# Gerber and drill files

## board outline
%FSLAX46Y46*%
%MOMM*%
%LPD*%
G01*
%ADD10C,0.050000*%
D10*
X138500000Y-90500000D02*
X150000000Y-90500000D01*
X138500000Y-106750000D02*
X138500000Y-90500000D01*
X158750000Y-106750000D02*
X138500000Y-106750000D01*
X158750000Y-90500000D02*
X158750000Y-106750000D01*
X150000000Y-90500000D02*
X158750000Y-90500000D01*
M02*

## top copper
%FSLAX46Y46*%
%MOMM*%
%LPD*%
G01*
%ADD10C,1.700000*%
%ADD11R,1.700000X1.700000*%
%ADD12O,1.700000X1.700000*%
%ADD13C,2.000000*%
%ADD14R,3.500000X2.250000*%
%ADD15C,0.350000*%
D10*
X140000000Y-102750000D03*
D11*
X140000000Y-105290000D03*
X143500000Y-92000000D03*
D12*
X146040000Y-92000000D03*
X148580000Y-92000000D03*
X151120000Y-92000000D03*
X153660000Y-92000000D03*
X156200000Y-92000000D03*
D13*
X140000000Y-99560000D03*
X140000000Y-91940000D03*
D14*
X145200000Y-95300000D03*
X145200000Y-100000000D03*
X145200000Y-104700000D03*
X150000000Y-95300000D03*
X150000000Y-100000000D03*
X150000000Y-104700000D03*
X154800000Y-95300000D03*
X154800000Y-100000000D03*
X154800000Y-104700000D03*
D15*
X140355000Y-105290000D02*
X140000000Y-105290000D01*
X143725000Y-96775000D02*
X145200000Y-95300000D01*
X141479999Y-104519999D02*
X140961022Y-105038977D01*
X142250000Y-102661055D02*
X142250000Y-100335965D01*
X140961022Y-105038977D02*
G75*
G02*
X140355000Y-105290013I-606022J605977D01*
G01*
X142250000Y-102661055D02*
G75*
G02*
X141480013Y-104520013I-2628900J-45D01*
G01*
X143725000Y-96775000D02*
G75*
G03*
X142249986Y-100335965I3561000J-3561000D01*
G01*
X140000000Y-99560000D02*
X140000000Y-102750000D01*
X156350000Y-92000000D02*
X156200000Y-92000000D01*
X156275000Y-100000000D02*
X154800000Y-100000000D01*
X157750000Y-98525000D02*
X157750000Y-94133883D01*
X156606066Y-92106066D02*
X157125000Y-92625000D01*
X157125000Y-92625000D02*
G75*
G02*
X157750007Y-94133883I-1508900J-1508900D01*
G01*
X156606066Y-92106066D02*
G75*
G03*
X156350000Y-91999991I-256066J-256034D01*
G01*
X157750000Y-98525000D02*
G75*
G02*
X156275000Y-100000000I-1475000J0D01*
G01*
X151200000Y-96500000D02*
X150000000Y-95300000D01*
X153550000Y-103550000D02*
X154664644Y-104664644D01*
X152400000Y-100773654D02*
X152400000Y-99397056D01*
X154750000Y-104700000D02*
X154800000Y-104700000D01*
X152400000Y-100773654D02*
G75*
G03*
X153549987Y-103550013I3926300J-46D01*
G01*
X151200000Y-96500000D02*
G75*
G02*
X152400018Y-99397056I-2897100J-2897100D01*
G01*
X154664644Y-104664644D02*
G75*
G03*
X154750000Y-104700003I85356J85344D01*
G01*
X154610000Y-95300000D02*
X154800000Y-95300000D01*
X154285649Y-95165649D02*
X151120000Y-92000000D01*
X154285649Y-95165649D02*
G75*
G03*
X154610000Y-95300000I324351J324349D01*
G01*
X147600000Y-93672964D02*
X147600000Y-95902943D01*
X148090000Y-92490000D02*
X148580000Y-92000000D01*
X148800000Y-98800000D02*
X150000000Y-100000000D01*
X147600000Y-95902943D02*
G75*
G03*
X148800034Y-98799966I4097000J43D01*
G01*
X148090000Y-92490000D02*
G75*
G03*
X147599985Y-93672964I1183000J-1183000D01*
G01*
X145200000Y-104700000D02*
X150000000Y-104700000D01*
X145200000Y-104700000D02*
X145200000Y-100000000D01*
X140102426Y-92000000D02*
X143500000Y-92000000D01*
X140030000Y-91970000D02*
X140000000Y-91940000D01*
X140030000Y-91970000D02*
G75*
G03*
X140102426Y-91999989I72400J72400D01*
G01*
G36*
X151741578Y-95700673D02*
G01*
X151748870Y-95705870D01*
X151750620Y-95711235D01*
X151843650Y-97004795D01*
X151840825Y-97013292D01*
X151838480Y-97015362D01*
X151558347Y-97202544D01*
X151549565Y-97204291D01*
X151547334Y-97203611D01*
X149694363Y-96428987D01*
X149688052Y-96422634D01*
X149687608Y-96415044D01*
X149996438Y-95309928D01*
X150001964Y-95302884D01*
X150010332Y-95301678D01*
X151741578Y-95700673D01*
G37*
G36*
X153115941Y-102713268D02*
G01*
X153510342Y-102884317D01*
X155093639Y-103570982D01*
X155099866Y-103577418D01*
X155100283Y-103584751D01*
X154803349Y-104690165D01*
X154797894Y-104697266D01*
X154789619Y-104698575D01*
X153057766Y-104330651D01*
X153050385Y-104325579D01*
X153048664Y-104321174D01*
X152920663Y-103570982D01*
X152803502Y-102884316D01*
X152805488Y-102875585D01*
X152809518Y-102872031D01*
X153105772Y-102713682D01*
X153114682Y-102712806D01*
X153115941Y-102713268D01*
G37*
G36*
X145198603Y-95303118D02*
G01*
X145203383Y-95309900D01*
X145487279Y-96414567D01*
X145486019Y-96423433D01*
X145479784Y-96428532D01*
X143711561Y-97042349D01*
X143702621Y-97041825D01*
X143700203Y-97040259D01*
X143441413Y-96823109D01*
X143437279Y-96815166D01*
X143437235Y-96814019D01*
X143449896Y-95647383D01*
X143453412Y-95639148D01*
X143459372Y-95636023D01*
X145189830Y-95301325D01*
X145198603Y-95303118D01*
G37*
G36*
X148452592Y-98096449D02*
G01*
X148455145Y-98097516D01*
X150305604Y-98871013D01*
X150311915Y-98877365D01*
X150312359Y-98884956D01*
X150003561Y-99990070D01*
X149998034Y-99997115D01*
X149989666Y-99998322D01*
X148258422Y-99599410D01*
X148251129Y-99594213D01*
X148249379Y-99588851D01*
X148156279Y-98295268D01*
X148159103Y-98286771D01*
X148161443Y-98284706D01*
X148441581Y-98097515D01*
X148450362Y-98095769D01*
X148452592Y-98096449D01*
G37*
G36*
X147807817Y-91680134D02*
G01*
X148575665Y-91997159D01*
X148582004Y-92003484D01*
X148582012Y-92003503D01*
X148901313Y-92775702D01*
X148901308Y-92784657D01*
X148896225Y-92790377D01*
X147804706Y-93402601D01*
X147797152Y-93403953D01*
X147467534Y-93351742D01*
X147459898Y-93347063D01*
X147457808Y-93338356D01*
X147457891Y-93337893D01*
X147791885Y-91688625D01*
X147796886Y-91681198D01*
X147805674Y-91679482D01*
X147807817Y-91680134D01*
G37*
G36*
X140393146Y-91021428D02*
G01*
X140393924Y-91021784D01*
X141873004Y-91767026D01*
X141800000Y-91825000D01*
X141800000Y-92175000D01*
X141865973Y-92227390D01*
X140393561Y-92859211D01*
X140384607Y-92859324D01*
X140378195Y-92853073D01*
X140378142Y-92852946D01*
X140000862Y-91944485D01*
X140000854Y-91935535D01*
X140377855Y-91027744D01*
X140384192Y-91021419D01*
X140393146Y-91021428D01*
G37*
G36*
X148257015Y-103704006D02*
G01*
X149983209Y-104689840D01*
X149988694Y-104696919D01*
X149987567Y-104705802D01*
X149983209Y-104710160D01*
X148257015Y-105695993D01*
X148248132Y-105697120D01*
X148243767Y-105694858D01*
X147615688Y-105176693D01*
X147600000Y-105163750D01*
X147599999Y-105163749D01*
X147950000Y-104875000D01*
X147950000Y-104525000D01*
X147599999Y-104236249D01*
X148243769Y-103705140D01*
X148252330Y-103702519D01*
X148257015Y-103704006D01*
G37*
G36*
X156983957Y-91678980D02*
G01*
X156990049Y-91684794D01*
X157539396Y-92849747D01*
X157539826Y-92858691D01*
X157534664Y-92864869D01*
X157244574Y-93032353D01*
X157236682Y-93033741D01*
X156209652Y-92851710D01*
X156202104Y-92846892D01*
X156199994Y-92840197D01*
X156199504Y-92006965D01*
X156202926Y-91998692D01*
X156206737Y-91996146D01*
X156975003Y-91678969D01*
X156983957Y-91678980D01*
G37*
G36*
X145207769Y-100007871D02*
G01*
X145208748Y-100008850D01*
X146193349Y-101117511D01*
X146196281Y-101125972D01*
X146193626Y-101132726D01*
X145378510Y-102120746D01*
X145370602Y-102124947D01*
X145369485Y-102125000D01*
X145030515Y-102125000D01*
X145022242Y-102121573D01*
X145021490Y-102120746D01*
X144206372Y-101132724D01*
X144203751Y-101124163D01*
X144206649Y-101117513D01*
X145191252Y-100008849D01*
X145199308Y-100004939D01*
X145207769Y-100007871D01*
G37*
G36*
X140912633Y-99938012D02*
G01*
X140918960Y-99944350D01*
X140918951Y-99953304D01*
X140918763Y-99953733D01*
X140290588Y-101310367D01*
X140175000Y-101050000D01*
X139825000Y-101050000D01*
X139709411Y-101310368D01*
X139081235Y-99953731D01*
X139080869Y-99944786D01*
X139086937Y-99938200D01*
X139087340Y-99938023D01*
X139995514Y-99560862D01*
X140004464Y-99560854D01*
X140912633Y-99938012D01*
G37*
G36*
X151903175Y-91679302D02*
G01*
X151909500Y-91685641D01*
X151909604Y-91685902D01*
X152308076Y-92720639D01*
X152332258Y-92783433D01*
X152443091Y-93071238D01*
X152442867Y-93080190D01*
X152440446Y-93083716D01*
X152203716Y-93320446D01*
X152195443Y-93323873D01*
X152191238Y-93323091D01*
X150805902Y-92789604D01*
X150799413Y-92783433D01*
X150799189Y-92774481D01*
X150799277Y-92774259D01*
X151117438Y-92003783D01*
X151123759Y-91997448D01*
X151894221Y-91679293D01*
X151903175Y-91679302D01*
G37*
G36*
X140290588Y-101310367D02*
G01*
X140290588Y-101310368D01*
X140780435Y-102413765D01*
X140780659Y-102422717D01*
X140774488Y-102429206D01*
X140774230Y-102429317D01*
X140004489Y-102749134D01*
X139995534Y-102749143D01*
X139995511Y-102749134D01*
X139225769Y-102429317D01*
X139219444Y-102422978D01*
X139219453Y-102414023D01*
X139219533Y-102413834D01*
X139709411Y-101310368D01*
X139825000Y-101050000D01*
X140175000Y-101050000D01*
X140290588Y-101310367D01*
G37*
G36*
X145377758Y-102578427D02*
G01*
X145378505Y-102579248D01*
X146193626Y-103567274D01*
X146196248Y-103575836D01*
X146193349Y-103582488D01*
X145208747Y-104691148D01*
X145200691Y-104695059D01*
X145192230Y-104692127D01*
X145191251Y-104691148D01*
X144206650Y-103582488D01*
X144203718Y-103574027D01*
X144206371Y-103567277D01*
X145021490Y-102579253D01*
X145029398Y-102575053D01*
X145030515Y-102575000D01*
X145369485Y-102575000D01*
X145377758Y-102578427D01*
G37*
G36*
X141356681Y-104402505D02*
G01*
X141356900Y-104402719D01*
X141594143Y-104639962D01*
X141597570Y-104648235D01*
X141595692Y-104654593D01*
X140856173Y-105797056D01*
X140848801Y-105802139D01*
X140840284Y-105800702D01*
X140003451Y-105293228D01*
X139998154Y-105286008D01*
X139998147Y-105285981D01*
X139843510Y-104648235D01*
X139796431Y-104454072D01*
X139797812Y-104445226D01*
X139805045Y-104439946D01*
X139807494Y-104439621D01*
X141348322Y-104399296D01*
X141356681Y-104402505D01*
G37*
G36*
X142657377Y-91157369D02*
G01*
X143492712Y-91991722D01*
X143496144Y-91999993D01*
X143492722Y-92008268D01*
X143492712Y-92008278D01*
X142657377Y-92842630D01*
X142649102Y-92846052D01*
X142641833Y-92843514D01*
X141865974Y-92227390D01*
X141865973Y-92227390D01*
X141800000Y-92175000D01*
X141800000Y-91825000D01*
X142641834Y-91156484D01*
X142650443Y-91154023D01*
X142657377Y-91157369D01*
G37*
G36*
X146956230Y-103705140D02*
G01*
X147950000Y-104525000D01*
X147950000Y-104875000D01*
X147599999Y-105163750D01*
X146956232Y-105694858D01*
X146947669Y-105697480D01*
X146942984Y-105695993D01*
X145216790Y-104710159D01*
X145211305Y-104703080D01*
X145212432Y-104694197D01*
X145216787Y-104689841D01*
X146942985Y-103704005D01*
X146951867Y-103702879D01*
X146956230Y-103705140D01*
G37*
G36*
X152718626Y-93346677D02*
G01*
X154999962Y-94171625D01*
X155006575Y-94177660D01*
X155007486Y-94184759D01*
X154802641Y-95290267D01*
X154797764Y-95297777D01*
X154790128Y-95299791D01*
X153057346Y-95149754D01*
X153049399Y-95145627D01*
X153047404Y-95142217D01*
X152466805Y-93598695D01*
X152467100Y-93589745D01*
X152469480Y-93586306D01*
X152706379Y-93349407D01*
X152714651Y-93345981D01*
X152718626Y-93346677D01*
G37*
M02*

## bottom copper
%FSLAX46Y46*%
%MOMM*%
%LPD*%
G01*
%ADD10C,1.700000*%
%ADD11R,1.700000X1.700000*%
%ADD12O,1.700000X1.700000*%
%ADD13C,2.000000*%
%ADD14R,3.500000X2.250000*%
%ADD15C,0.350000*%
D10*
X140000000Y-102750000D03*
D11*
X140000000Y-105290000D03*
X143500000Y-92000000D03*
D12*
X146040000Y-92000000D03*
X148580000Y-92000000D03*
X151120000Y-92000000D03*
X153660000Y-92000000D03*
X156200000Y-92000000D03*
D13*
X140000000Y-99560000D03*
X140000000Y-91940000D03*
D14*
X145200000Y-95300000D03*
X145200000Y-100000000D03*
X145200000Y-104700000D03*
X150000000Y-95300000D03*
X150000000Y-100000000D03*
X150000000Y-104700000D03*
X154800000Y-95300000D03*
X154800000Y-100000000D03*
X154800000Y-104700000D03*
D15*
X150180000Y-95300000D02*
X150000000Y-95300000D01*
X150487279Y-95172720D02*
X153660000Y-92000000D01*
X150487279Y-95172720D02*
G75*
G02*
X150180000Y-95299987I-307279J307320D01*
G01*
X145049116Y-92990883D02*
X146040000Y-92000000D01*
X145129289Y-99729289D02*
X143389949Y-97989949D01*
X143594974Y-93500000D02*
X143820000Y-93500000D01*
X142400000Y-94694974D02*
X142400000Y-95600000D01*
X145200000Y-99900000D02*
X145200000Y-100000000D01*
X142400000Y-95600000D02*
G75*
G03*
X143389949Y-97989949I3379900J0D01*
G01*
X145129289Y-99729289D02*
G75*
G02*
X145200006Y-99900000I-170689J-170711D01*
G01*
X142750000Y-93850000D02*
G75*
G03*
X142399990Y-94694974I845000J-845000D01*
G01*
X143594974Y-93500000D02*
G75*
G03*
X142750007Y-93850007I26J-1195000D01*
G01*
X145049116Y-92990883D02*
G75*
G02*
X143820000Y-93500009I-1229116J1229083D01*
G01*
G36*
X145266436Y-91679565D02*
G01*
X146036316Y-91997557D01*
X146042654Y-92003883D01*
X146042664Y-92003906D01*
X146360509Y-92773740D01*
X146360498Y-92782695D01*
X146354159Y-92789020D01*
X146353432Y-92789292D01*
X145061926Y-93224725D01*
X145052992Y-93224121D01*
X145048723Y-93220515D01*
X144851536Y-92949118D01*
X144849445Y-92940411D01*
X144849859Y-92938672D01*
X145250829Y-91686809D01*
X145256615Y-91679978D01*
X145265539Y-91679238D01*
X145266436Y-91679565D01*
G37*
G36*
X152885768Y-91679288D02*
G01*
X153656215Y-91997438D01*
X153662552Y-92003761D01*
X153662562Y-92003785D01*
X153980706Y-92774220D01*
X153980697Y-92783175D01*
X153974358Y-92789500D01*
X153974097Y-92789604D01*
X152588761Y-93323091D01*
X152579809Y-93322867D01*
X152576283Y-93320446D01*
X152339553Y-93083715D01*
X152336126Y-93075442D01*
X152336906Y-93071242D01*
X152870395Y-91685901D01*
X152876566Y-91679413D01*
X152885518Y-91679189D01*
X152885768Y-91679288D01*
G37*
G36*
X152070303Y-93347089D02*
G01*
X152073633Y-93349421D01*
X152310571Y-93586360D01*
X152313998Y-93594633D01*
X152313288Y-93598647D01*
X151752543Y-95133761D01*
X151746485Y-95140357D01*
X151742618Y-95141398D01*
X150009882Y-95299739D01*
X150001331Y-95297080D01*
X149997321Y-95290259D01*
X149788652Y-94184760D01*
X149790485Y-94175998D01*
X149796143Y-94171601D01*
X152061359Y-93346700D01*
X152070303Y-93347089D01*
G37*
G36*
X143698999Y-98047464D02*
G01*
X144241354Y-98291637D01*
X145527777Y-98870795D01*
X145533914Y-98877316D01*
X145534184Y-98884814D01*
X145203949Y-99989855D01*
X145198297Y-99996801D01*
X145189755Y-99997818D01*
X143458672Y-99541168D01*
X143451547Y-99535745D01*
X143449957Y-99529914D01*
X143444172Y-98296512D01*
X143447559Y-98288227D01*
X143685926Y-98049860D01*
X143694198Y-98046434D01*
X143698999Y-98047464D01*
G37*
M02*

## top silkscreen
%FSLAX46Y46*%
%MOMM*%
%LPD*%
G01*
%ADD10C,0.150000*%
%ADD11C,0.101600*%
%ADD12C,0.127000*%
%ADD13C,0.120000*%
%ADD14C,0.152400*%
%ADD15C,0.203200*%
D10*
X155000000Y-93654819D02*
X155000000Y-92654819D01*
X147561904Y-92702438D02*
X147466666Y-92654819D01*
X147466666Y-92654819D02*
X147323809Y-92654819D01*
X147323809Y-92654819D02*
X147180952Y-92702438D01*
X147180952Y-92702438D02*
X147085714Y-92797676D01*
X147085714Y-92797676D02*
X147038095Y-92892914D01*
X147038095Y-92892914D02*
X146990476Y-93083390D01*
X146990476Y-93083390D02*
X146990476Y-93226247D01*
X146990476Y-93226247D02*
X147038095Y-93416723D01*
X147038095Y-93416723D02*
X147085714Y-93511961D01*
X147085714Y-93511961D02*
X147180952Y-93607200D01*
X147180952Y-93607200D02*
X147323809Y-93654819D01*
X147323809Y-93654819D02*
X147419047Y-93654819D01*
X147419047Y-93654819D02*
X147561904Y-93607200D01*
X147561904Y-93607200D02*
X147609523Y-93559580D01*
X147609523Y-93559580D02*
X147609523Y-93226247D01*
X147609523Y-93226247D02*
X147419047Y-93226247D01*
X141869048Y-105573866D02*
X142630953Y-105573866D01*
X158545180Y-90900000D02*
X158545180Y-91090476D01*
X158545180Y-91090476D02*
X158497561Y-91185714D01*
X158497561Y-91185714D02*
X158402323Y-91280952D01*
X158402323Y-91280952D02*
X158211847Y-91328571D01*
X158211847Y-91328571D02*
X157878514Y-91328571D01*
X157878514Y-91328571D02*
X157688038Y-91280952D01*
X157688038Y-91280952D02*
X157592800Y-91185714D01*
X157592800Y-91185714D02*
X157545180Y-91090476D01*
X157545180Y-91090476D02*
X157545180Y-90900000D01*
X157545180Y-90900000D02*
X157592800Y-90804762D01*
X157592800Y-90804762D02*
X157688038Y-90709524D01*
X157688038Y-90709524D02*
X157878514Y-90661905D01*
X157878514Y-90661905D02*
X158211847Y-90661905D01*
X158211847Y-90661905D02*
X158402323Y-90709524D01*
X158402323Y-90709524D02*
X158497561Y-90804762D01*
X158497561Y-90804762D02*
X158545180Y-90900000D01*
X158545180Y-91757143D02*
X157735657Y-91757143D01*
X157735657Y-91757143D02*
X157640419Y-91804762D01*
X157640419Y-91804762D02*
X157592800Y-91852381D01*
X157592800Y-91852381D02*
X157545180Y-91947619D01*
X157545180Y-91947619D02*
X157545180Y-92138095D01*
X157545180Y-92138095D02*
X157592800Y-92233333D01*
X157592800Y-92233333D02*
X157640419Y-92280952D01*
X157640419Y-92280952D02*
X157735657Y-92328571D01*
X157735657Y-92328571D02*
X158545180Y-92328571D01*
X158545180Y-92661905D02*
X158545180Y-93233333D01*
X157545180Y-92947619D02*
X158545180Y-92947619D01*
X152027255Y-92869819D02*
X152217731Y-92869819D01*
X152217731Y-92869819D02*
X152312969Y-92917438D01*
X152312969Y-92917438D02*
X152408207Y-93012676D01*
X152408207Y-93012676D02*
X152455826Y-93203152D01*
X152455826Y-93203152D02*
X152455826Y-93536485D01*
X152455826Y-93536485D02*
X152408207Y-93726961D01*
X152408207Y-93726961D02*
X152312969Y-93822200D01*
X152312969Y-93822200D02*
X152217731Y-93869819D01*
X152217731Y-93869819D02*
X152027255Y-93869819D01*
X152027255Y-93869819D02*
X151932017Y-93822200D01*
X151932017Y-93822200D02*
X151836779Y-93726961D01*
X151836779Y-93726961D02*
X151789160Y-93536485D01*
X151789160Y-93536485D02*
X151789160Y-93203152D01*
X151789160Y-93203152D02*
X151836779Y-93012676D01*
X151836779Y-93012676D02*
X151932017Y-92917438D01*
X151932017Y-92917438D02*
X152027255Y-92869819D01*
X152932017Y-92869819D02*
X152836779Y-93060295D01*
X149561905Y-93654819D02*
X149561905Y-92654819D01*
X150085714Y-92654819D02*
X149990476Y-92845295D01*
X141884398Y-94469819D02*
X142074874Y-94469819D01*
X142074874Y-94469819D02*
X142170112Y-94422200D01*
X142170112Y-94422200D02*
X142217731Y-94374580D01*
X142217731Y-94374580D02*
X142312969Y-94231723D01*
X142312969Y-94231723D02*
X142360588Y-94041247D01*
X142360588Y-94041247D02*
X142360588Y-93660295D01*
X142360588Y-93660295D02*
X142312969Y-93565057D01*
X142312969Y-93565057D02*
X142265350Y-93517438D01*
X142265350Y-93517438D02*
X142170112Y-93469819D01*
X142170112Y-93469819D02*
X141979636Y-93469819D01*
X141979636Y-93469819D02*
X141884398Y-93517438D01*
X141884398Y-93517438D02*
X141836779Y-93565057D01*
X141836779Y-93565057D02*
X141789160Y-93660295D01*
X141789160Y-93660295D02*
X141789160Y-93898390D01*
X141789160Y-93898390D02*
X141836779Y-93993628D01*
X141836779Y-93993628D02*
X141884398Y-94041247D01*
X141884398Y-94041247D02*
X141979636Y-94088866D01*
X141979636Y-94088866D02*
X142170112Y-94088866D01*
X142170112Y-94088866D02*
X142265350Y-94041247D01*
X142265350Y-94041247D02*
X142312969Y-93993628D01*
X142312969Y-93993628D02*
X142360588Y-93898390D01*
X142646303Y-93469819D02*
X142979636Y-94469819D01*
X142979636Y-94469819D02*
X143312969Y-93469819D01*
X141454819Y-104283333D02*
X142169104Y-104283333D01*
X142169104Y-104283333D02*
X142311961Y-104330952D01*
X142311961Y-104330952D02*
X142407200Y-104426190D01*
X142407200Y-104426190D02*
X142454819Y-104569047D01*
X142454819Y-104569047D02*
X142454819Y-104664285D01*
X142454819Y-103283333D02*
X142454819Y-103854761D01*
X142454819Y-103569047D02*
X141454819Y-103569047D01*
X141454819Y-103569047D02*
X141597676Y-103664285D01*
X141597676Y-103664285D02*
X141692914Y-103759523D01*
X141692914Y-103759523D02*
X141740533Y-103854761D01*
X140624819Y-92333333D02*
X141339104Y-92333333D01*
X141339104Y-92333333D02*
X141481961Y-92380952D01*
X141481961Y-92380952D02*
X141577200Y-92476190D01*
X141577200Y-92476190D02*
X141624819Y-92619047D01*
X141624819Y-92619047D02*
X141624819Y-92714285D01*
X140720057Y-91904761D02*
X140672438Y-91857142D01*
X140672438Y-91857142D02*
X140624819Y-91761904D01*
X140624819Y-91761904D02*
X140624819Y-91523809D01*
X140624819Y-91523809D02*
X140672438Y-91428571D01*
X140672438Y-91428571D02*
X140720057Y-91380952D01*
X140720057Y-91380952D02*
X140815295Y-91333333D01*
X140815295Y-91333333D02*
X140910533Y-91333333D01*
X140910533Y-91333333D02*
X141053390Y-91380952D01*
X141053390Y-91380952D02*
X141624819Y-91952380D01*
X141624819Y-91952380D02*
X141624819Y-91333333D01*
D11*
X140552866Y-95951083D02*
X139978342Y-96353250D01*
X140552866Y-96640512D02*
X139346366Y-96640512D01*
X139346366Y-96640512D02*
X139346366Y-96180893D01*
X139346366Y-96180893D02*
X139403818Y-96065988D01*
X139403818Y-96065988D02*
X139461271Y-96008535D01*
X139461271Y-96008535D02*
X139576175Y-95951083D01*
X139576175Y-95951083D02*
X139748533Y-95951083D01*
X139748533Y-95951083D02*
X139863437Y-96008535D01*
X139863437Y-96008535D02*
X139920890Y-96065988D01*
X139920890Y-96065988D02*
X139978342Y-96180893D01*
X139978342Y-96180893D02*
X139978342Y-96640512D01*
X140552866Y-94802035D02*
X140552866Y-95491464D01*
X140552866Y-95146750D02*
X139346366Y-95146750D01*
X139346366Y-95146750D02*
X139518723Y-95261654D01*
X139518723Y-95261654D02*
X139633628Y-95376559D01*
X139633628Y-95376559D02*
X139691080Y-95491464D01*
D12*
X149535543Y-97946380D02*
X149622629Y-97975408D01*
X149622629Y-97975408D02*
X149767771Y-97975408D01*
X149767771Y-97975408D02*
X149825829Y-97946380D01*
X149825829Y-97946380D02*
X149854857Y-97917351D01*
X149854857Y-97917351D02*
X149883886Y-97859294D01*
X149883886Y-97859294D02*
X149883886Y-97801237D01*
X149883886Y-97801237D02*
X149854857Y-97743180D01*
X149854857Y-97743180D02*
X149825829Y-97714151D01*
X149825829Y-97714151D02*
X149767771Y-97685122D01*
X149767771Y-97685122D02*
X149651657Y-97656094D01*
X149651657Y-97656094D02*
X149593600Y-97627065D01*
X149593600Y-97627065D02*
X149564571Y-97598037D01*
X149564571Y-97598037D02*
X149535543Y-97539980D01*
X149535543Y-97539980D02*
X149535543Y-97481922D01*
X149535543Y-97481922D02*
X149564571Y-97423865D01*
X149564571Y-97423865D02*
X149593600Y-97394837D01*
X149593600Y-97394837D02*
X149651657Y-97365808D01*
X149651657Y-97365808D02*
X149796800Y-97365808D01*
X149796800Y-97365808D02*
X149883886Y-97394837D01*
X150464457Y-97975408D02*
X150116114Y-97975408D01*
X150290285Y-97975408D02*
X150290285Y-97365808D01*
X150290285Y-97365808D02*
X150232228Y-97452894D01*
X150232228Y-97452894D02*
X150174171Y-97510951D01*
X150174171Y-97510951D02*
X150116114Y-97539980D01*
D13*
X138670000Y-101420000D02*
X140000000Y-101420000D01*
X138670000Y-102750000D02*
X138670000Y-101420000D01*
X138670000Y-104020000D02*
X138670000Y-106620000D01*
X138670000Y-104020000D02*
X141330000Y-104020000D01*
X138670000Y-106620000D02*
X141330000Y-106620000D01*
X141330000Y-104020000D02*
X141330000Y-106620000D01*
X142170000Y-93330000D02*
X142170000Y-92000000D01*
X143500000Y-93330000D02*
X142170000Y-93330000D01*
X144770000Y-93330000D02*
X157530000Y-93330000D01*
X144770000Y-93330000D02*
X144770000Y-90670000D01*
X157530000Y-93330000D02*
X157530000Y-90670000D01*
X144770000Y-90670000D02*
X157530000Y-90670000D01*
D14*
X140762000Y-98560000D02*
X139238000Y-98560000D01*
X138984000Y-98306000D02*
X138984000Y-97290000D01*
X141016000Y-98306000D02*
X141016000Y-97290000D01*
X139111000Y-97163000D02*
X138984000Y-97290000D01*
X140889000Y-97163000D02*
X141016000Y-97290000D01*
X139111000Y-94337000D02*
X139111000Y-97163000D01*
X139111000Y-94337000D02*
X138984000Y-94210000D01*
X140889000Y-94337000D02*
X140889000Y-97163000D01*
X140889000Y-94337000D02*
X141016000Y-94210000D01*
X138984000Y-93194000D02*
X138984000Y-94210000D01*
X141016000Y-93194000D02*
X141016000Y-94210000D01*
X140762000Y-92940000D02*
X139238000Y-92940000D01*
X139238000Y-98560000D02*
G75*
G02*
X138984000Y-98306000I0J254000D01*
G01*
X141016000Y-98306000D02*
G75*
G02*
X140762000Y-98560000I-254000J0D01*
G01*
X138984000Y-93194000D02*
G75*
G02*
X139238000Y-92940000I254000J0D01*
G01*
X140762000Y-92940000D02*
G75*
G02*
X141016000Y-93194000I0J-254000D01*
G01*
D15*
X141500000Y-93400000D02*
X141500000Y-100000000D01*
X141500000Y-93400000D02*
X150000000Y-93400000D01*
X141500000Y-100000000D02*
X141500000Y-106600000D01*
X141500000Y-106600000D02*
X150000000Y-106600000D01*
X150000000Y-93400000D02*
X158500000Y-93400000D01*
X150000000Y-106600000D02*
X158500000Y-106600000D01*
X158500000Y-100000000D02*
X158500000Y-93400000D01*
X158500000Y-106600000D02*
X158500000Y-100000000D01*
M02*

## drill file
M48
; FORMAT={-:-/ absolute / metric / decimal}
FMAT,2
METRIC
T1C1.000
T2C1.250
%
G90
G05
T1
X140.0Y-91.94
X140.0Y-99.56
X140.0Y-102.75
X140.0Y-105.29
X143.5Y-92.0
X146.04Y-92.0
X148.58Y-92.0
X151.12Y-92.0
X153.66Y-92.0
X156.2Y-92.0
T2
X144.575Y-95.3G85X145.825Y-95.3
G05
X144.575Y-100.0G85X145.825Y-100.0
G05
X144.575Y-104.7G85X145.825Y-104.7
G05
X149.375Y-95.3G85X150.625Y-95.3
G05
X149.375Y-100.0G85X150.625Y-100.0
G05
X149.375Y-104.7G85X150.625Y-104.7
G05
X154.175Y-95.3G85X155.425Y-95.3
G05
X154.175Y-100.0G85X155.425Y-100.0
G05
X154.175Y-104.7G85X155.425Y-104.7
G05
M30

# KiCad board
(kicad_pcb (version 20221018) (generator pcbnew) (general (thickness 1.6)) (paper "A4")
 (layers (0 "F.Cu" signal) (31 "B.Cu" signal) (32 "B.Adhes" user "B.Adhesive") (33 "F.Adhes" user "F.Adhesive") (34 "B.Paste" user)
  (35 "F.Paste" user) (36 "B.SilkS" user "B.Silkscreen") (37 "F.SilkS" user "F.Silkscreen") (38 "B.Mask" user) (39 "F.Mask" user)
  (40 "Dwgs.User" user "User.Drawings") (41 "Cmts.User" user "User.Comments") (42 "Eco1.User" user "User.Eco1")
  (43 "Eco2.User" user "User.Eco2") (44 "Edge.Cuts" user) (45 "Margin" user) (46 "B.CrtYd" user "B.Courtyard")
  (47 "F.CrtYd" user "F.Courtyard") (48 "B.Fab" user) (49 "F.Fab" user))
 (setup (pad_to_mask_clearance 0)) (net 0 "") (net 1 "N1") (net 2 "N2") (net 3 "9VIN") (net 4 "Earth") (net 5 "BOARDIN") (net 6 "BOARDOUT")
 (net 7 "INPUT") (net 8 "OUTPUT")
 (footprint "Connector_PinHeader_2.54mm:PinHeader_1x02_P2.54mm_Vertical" (layer "F.Cu") (at 140 102.75)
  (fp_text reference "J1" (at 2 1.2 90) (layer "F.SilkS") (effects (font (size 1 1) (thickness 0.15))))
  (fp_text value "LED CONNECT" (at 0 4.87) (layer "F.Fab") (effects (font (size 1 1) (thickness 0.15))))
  (fp_line (start -1.33 -1.33) (end 0 -1.33) (stroke (width 0.12) (type solid)) (layer "F.SilkS"))
  (fp_line (start -1.33 0) (end -1.33 -1.33) (stroke (width 0.12) (type solid)) (layer "F.SilkS"))
  (fp_line (start -1.33 1.27) (end -1.33 3.87) (stroke (width 0.12) (type solid)) (layer "F.SilkS"))
  (fp_line (start -1.33 1.27) (end 1.33 1.27) (stroke (width 0.12) (type solid)) (layer "F.SilkS"))
  (fp_line (start -1.33 3.87) (end 1.33 3.87) (stroke (width 0.12) (type solid)) (layer "F.SilkS"))
  (fp_line (start 1.33 1.27) (end 1.33 3.87) (stroke (width 0.12) (type solid)) (layer "F.SilkS"))
  (pad "1" thru_hole circle (at 0 0) (size 1.7 1.7) (drill 1) (layers "*.Cu" "*.Mask") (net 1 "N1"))
  (pad "2" thru_hole rect (at 0 2.54) (size 1.7 1.7) (drill 1) (layers "*.Cu" "*.Mask") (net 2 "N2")))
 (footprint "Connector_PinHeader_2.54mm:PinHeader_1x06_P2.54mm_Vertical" (layer "F.Cu") (at 143.5 92 90)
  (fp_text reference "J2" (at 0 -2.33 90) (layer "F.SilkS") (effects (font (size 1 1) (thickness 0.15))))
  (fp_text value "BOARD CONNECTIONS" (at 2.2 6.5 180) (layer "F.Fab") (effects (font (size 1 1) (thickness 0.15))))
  (fp_line (start -1.33 -1.33) (end 0 -1.33) (stroke (width 0.12) (type solid)) (layer "F.SilkS"))
  (fp_line (start -1.33 0) (end -1.33 -1.33) (stroke (width 0.12) (type solid)) (layer "F.SilkS"))
  (fp_line (start -1.33 1.27) (end -1.33 14.03) (stroke (width 0.12) (type solid)) (layer "F.SilkS"))
  (fp_line (start -1.33 1.27) (end 1.33 1.27) (stroke (width 0.12) (type solid)) (layer "F.SilkS"))
  (fp_line (start -1.33 14.03) (end 1.33 14.03) (stroke (width 0.12) (type solid)) (layer "F.SilkS"))
  (fp_line (start 1.33 1.27) (end 1.33 14.03) (stroke (width 0.12) (type solid)) (layer "F.SilkS"))
  (pad "1" thru_hole rect (at 0 0 90) (size 1.7 1.7) (drill 1) (layers "*.Cu" "*.Mask") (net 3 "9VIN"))
  (pad "2" thru_hole oval (at 0 2.54 90) (size 1.7 1.7) (drill 1) (layers "*.Cu" "*.Mask") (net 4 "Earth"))
  (pad "3" thru_hole oval (at 0 5.08 90) (size 1.7 1.7) (drill 1) (layers "*.Cu" "*.Mask") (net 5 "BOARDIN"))
  (pad "4" thru_hole oval (at 0 7.62 90) (size 1.7 1.7) (drill 1) (layers "*.Cu" "*.Mask") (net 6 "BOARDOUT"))
  (pad "5" thru_hole oval (at 0 10.16 90) (size 1.7 1.7) (drill 1) (layers "*.Cu" "*.Mask") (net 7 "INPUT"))
  (pad "6" thru_hole oval (at 0 12.7 90) (size 1.7 1.7) (drill 1) (layers "*.Cu" "*.Mask") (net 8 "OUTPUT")))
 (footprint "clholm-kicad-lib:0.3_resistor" (layer "F.Cu") (at 140 95.75 90)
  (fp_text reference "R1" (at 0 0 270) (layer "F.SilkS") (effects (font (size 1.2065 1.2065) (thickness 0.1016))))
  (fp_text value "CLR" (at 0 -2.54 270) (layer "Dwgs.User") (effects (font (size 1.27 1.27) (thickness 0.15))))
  (fp_line (start -2.81 0.762) (end -2.81 -0.762) (stroke (width 0.1524) (type solid)) (layer "F.SilkS"))
  (fp_line (start -2.556 -1.016) (end -1.54 -1.016) (stroke (width 0.1524) (type solid)) (layer "F.SilkS"))
  (fp_line (start -2.556 1.016) (end -1.54 1.016) (stroke (width 0.1524) (type solid)) (layer "F.SilkS"))
  (fp_line (start -1.413 -0.889) (end -1.54 -1.016) (stroke (width 0.1524) (type solid)) (layer "F.SilkS"))
  (fp_line (start -1.413 0.889) (end -1.54 1.016) (stroke (width 0.1524) (type solid)) (layer "F.SilkS"))
  (fp_line (start 1.413 -0.889) (end -1.413 -0.889) (stroke (width 0.1524) (type solid)) (layer "F.SilkS"))
  (fp_line (start 1.413 -0.889) (end 1.54 -1.016) (stroke (width 0.1524) (type solid)) (layer "F.SilkS"))
  (fp_line (start 1.413 0.889) (end -1.413 0.889) (stroke (width 0.1524) (type solid)) (layer "F.SilkS"))
  (fp_line (start 1.413 0.889) (end 1.54 1.016) (stroke (width 0.1524) (type solid)) (layer "F.SilkS"))
  (fp_line (start 2.556 -1.016) (end 1.54 -1.016) (stroke (width 0.1524) (type solid)) (layer "F.SilkS"))
  (fp_line (start 2.556 1.016) (end 1.54 1.016) (stroke (width 0.1524) (type solid)) (layer "F.SilkS"))
  (fp_line (start 2.81 0.762) (end 2.81 -0.762) (stroke (width 0.1524) (type solid)) (layer "F.SilkS"))
  (fp_arc (start -2.81 -0.762) (mid -2.735605 -0.941605) (end -2.556 -1.016) (stroke (width 0.1524) (type solid)) (layer "F.SilkS"))
  (fp_arc (start -2.556 1.016) (mid -2.735605 0.941605) (end -2.81 0.762) (stroke (width 0.1524) (type solid)) (layer "F.SilkS"))
  (fp_arc (start 2.556 -1.016) (mid 2.735605 -0.941605) (end 2.81 -0.762) (stroke (width 0.1524) (type solid)) (layer "F.SilkS"))
  (fp_arc (start 2.81 0.762) (mid 2.735605 0.941605) (end 2.556 1.016) (stroke (width 0.1524) (type solid)) (layer "F.SilkS"))
  (pad "1" thru_hole circle (at -3.81 0 90) (size 2 2) (drill 1) (layers "*.Cu" "*.Mask") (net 1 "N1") (solder_mask_margin 0.1016))
  (pad "2" thru_hole circle (at 3.81 0 90) (size 2 2) (drill 1) (layers "*.Cu" "*.Mask") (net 3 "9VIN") (solder_mask_margin 0.1016)))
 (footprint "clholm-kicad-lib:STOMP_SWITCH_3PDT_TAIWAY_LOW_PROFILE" (layer "F.Cu") (at 150 100)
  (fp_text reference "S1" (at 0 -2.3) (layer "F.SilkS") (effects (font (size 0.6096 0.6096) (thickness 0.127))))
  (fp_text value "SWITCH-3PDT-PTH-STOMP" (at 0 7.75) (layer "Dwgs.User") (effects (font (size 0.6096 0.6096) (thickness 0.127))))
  (fp_line (start -8.5 -6.6) (end -8.5 0) (stroke (width 0.2032) (type solid)) (layer "F.SilkS"))
  (fp_line (start -8.5 -6.6) (end 0 -6.6) (stroke (width 0.2032) (type solid)) (layer "F.SilkS"))
  (fp_line (start -8.5 0) (end -8.5 6.6) (stroke (width 0.2032) (type solid)) (layer "F.SilkS"))
  (fp_line (start -8.5 6.6) (end 0 6.6) (stroke (width 0.2032) (type solid)) (layer "F.SilkS"))
  (fp_line (start 0 -6.6) (end 8.5 -6.6) (stroke (width 0.2032) (type solid)) (layer "F.SilkS"))
  (fp_line (start 0 6.6) (end 8.5 6.6) (stroke (width 0.2032) (type solid)) (layer "F.SilkS"))
  (fp_line (start 8.5 0) (end 8.5 -6.6) (stroke (width 0.2032) (type solid)) (layer "F.SilkS"))
  (fp_line (start 8.5 6.6) (end 8.5 0) (stroke (width 0.2032) (type solid)) (layer "F.SilkS"))
  (pad "P$1" thru_hole rect (at -4.8 -4.7) (size 3.5 2.25) (drill oval 2.5 1.25) (layers "*.Cu" "*.Mask") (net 2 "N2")
   (solder_mask_margin 0.1016))
  (pad "P$2" thru_hole rect (at -4.8 0) (size 3.5 2.25) (drill oval 2.5 1.25) (layers "*.Cu" "*.Mask") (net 4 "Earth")
   (solder_mask_margin 0.1016))
  (pad "P$3" thru_hole rect (at -4.8 4.7) (size 3.5 2.25) (drill oval 2.5 1.25) (layers "*.Cu" "*.Mask") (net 4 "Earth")
   (solder_mask_margin 0.1016))
  (pad "P$4" thru_hole rect (at 0 -4.7) (size 3.5 2.25) (drill oval 2.5 1.25) (layers "*.Cu" "*.Mask") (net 7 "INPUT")
   (solder_mask_margin 0.1016))
  (pad "P$5" thru_hole rect (at 0 0) (size 3.5 2.25) (drill oval 2.5 1.25) (layers "*.Cu" "*.Mask") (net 5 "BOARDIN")
   (solder_mask_margin 0.1016))
  (pad "P$6" thru_hole rect (at 0 4.7) (size 3.5 2.25) (drill oval 2.5 1.25) (layers "*.Cu" "*.Mask") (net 4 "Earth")
   (solder_mask_margin 0.1016))
  (pad "P$7" thru_hole rect (at 4.8 -4.7) (size 3.5 2.25) (drill oval 2.5 1.25) (layers "*.Cu" "*.Mask") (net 6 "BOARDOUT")
   (solder_mask_margin 0.1016))
  (pad "P$8" thru_hole rect (at 4.8 0) (size 3.5 2.25) (drill oval 2.5 1.25) (layers "*.Cu" "*.Mask") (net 8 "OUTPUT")
   (solder_mask_margin 0.1016))
  (pad "P$9" thru_hole rect (at 4.8 4.7) (size 3.5 2.25) (drill oval 2.5 1.25) (layers "*.Cu" "*.Mask") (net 7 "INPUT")
   (solder_mask_margin 0.1016)))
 (gr_line (start 138.5 90.5) (end 150 90.5) (stroke (width 0.05) (type solid)) (layer "Edge.Cuts"))
 (gr_line (start 138.5 106.75) (end 138.5 90.5) (stroke (width 0.05) (type solid)) (layer "Edge.Cuts"))
 (gr_line (start 158.75 106.75) (end 138.5 106.75) (stroke (width 0.05) (type solid)) (layer "Edge.Cuts"))
 (gr_line (start 158.75 90.5) (end 158.75 106.75) (stroke (width 0.05) (type solid)) (layer "Edge.Cuts"))
 (gr_line (start 150 90.5) (end 158.75 90.5) (stroke (width 0.05) (type solid)) (layer "Edge.Cuts"))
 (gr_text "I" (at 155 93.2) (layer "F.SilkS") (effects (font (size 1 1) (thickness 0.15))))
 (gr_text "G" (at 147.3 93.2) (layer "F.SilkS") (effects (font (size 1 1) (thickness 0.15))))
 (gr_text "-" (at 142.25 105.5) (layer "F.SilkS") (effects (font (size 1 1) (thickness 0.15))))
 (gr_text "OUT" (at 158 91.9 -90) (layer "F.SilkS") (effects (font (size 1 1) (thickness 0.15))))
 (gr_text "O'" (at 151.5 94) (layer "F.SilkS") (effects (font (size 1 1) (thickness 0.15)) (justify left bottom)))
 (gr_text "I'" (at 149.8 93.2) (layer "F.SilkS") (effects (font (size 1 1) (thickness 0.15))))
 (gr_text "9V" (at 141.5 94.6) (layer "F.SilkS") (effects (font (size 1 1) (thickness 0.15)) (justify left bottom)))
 (segment (start 140.355 105.29) (end 140 105.29) (width 0.35) (layer "F.Cu") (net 2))
 (segment (start 143.725 96.775) (end 145.2 95.3) (width 0.35) (layer "F.Cu") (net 2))
 (segment (start 141.479999 104.519999) (end 140.961022 105.038977) (width 0.35) (layer "F.Cu") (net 2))
 (segment (start 142.25 102.661055) (end 142.25 100.335965) (width 0.35) (layer "F.Cu") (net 2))
 (arc (start 140.961022 105.038977) (mid 140.682976 105.224761) (end 140.355 105.29) (width 0.35) (layer "F.Cu") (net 2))
 (arc (start 142.25 102.661055) (mid 142.049883 103.667108) (end 141.479999 104.519999) (width 0.35) (layer "F.Cu") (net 2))
 (arc (start 143.725 96.775) (mid 142.63334 98.408784) (end 142.25 100.335965) (width 0.35) (layer "F.Cu") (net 2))
 (segment (start 140 99.56) (end 140 102.75) (width 0.35) (layer "F.Cu") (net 1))
 (segment (start 156.35 92) (end 156.2 92) (width 0.35) (layer "F.Cu") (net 8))
 (segment (start 156.275 100) (end 154.8 100) (width 0.35) (layer "F.Cu") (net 8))
 (segment (start 157.75 98.525) (end 157.75 94.133883) (width 0.35) (layer "F.Cu") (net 8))
 (segment (start 156.606066 92.106066) (end 157.125 92.625) (width 0.35) (layer "F.Cu") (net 8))
 (arc (start 157.125 92.625) (mid 157.587567 93.317281) (end 157.75 94.133883) (width 0.35) (layer "F.Cu") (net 8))
 (arc (start 156.606066 92.106066) (mid 156.488581 92.027565) (end 156.35 92) (width 0.35) (layer "F.Cu") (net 8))
 (arc (start 157.75 98.525) (mid 157.317982 99.567982) (end 156.275 100) (width 0.35) (layer "F.Cu") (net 8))
 (segment (start 151.2 96.5) (end 150 95.3) (width 0.35) (layer "F.Cu") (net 7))
 (segment (start 153.55 103.55) (end 154.664644 104.664644) (width 0.35) (layer "F.Cu") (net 7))
 (segment (start 152.4 100.773654) (end 152.4 99.397056) (width 0.35) (layer "F.Cu") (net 7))
 (segment (start 154.75 104.7) (end 154.8 104.7) (width 0.35) (layer "F.Cu") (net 7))
 (arc (start 152.4 100.773654) (mid 152.698875 102.276201) (end 153.55 103.55) (width 0.35) (layer "F.Cu") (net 7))
 (arc (start 151.2 96.5) (mid 152.08813 97.82918) (end 152.4 99.397056) (width 0.35) (layer "F.Cu") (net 7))
 (arc (start 154.664644 104.664644) (mid 154.703805 104.690811) (end 154.75 104.7) (width 0.35) (layer "F.Cu") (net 7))
 (segment (start 150.18 95.3) (end 150 95.3) (width 0.35) (layer "B.Cu") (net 7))
 (segment (start 150.487279 95.17272) (end 153.66 92) (width 0.35) (layer "B.Cu") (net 7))
 (arc (start 150.487279 95.17272) (mid 150.346298 95.266921) (end 150.18 95.3) (width 0.35) (layer "B.Cu") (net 7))
 (segment (start 154.61 95.3) (end 154.8 95.3) (width 0.35) (layer "F.Cu") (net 6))
 (segment (start 154.285649 95.165649) (end 151.12 92) (width 0.35) (layer "F.Cu") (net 6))
 (arc (start 154.285649 95.165649) (mid 154.434462 95.265083) (end 154.61 95.3) (width 0.35) (layer "F.Cu") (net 6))
 (segment (start 147.6 93.672964) (end 147.6 95.902943) (width 0.35) (layer "F.Cu") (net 5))
 (segment (start 148.09 92.49) (end 148.58 92) (width 0.35) (layer "F.Cu") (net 5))
 (segment (start 148.8 98.8) (end 150 100) (width 0.35) (layer "F.Cu") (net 5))
 (arc (start 147.6 95.902943) (mid 147.911869 97.470819) (end 148.8 98.8) (width 0.35) (layer "F.Cu") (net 5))
 (arc (start 148.09 92.49) (mid 147.727346 93.032748) (end 147.6 93.672964) (width 0.35) (layer "F.Cu") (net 5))
 (segment (start 145.2 104.7) (end 150 104.7) (width 0.35) (layer "F.Cu") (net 4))
 (segment (start 145.2 104.7) (end 145.2 100) (width 0.35) (layer "F.Cu") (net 4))
 (segment (start 145.049116 92.990883) (end 146.04 92) (width 0.35) (layer "B.Cu") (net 4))
 (segment (start 145.129289 99.729289) (end 143.389949 97.989949) (width 0.35) (layer "B.Cu") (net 4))
 (segment (start 143.594974 93.5) (end 143.82 93.5) (width 0.35) (layer "B.Cu") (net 4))
 (segment (start 142.4 94.694974) (end 142.4 95.6) (width 0.35) (layer "B.Cu") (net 4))
 (segment (start 145.2 99.9) (end 145.2 100) (width 0.35) (layer "B.Cu") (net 4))
 (arc (start 142.4 95.6) (mid 142.657279 96.893431) (end 143.389949 97.989949) (width 0.35) (layer "B.Cu") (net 4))
 (arc (start 145.129289 99.729289) (mid 145.181622 99.807611) (end 145.2 99.9) (width 0.35) (layer "B.Cu") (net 4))
 (arc (start 142.75 93.85) (mid 142.490962 94.237677) (end 142.4 94.694974) (width 0.35) (layer "B.Cu") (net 4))
 (arc (start 143.594974 93.5) (mid 143.137677 93.590962) (end 142.75 93.85) (width 0.35) (layer "B.Cu") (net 4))
 (arc (start 145.049116 92.990883) (mid 144.485193 93.367684) (end 143.82 93.5) (width 0.35) (layer "B.Cu") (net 4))
 (segment (start 140.102426 92) (end 143.5 92) (width 0.35) (layer "F.Cu") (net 3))
 (segment (start 140.03 91.97) (end 140 91.94) (width 0.35) (layer "F.Cu") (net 3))
 (arc (start 140.03 91.97) (mid 140.063229 91.992203) (end 140.102426 92) (width 0.35) (layer "F.Cu") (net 3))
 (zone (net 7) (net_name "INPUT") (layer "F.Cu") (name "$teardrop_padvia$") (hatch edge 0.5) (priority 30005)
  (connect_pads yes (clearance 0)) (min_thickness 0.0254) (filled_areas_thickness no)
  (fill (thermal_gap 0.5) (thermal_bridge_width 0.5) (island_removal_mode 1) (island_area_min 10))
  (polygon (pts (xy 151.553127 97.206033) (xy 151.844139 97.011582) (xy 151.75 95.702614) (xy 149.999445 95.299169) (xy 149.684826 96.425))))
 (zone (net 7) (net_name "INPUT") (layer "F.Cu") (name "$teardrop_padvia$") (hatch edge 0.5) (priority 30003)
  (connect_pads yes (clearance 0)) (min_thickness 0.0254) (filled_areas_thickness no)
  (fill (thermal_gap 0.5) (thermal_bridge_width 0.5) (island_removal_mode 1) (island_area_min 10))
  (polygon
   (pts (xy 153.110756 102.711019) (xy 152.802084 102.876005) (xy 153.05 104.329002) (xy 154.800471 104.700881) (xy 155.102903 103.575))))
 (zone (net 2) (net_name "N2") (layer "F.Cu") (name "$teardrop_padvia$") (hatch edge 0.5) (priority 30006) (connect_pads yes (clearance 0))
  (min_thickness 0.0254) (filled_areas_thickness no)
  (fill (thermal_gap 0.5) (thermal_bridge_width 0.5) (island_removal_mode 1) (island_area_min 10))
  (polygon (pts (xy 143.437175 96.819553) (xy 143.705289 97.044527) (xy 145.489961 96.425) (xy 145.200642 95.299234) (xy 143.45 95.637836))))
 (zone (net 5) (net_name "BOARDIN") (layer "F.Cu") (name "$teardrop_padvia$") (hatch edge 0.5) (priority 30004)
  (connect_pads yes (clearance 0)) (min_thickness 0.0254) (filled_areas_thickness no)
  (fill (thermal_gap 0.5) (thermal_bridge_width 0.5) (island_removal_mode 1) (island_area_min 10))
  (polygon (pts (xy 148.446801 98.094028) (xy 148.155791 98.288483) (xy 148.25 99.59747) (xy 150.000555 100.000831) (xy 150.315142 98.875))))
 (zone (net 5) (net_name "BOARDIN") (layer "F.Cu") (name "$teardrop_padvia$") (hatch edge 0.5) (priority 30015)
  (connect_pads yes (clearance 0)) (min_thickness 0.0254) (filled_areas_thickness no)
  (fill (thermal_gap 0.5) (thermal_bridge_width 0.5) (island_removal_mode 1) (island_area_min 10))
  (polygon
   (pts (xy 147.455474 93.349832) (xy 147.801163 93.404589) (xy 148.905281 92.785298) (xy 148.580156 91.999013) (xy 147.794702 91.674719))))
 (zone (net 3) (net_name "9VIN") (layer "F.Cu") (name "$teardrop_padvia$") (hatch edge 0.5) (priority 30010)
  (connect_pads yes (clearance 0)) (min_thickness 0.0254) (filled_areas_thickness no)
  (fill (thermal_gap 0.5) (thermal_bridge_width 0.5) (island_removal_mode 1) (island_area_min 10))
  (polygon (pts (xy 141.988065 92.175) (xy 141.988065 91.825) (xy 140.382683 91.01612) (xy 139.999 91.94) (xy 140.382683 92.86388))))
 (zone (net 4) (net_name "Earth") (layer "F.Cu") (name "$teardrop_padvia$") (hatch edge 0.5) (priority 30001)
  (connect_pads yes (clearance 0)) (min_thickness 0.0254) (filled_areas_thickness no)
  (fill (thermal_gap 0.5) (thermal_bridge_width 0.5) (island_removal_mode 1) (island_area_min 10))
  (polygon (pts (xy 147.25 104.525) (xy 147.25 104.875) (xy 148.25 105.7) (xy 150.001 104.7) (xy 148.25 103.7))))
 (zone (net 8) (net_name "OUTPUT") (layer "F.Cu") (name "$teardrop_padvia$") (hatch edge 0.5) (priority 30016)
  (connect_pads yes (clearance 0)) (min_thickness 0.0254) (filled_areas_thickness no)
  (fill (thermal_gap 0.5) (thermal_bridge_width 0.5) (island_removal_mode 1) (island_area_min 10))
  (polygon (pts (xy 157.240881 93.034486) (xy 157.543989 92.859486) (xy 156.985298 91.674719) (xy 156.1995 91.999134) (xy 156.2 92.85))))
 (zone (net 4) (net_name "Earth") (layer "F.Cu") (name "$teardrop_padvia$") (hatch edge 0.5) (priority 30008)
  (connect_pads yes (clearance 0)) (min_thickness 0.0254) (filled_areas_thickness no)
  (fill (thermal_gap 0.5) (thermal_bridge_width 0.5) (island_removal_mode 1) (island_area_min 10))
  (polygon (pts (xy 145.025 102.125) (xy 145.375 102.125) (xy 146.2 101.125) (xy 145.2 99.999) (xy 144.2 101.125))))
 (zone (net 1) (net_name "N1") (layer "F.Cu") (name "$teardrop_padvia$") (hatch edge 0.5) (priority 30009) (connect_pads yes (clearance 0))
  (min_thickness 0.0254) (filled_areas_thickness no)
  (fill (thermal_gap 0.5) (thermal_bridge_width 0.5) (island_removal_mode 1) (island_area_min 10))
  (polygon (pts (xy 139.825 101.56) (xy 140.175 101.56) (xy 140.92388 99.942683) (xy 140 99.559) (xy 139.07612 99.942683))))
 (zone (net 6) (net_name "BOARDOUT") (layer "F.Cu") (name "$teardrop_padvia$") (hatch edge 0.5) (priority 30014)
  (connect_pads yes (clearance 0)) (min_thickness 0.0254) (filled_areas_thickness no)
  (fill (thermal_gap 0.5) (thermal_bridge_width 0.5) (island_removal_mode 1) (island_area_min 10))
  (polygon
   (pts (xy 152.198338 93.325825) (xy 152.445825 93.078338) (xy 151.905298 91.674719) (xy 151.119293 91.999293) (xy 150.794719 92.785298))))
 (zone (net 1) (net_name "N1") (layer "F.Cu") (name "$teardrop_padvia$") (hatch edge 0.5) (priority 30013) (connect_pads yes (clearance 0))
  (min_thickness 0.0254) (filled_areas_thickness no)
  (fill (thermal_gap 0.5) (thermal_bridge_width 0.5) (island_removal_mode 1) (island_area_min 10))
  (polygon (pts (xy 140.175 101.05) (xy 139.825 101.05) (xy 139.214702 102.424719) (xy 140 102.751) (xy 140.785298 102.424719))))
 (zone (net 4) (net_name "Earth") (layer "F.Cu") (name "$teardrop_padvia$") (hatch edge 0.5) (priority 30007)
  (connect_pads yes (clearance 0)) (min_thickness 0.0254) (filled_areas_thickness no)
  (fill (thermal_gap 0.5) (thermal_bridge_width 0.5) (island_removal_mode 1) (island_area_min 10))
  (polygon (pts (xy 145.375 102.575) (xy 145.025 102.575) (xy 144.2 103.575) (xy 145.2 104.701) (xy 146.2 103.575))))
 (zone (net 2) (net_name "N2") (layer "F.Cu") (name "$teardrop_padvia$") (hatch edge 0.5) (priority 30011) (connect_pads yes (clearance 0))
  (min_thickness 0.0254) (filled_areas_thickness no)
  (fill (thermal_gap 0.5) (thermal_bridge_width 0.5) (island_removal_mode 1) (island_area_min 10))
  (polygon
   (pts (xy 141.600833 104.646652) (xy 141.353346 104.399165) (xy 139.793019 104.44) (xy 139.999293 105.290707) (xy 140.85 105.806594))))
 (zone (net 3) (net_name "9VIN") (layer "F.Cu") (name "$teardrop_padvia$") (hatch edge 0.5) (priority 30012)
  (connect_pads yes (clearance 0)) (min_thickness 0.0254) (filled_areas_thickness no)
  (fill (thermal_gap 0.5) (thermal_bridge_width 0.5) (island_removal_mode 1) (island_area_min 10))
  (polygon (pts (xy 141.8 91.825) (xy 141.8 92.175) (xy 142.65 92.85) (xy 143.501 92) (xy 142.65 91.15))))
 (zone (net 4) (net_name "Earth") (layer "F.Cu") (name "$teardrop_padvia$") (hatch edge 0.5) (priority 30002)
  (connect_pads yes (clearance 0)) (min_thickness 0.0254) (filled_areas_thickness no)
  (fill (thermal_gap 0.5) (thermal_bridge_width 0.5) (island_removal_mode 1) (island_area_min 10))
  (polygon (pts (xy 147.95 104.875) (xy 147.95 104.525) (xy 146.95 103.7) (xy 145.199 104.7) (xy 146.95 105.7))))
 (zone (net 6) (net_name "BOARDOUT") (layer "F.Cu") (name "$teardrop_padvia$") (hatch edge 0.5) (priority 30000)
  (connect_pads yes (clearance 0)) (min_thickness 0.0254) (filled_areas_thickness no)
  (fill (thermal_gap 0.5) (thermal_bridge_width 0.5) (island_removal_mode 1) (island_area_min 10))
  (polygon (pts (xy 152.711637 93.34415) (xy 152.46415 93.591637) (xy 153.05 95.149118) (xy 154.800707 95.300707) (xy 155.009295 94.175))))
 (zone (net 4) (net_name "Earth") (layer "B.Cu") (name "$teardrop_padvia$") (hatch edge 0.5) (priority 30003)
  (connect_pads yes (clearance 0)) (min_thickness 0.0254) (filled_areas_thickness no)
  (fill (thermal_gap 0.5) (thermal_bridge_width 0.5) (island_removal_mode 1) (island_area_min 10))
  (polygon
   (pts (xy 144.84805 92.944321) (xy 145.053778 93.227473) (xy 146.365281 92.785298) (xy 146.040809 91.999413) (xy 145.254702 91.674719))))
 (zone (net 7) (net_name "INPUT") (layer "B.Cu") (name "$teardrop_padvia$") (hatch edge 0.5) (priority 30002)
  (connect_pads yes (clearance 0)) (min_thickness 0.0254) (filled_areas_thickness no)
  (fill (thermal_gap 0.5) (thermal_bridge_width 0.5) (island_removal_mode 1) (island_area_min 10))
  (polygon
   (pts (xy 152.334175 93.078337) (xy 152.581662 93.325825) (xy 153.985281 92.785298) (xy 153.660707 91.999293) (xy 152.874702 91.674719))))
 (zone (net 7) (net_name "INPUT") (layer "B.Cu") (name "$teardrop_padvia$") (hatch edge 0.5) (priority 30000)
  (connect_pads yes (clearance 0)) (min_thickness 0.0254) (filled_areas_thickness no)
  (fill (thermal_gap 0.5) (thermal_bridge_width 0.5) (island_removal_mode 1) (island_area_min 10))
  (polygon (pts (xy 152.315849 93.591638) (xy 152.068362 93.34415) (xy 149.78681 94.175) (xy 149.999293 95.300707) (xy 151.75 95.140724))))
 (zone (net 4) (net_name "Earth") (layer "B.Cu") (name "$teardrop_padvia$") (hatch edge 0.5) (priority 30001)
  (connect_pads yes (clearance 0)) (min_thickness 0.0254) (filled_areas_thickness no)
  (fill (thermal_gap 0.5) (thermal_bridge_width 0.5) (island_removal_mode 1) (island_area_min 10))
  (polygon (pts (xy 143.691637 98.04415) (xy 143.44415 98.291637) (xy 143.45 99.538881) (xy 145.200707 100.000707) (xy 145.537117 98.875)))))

